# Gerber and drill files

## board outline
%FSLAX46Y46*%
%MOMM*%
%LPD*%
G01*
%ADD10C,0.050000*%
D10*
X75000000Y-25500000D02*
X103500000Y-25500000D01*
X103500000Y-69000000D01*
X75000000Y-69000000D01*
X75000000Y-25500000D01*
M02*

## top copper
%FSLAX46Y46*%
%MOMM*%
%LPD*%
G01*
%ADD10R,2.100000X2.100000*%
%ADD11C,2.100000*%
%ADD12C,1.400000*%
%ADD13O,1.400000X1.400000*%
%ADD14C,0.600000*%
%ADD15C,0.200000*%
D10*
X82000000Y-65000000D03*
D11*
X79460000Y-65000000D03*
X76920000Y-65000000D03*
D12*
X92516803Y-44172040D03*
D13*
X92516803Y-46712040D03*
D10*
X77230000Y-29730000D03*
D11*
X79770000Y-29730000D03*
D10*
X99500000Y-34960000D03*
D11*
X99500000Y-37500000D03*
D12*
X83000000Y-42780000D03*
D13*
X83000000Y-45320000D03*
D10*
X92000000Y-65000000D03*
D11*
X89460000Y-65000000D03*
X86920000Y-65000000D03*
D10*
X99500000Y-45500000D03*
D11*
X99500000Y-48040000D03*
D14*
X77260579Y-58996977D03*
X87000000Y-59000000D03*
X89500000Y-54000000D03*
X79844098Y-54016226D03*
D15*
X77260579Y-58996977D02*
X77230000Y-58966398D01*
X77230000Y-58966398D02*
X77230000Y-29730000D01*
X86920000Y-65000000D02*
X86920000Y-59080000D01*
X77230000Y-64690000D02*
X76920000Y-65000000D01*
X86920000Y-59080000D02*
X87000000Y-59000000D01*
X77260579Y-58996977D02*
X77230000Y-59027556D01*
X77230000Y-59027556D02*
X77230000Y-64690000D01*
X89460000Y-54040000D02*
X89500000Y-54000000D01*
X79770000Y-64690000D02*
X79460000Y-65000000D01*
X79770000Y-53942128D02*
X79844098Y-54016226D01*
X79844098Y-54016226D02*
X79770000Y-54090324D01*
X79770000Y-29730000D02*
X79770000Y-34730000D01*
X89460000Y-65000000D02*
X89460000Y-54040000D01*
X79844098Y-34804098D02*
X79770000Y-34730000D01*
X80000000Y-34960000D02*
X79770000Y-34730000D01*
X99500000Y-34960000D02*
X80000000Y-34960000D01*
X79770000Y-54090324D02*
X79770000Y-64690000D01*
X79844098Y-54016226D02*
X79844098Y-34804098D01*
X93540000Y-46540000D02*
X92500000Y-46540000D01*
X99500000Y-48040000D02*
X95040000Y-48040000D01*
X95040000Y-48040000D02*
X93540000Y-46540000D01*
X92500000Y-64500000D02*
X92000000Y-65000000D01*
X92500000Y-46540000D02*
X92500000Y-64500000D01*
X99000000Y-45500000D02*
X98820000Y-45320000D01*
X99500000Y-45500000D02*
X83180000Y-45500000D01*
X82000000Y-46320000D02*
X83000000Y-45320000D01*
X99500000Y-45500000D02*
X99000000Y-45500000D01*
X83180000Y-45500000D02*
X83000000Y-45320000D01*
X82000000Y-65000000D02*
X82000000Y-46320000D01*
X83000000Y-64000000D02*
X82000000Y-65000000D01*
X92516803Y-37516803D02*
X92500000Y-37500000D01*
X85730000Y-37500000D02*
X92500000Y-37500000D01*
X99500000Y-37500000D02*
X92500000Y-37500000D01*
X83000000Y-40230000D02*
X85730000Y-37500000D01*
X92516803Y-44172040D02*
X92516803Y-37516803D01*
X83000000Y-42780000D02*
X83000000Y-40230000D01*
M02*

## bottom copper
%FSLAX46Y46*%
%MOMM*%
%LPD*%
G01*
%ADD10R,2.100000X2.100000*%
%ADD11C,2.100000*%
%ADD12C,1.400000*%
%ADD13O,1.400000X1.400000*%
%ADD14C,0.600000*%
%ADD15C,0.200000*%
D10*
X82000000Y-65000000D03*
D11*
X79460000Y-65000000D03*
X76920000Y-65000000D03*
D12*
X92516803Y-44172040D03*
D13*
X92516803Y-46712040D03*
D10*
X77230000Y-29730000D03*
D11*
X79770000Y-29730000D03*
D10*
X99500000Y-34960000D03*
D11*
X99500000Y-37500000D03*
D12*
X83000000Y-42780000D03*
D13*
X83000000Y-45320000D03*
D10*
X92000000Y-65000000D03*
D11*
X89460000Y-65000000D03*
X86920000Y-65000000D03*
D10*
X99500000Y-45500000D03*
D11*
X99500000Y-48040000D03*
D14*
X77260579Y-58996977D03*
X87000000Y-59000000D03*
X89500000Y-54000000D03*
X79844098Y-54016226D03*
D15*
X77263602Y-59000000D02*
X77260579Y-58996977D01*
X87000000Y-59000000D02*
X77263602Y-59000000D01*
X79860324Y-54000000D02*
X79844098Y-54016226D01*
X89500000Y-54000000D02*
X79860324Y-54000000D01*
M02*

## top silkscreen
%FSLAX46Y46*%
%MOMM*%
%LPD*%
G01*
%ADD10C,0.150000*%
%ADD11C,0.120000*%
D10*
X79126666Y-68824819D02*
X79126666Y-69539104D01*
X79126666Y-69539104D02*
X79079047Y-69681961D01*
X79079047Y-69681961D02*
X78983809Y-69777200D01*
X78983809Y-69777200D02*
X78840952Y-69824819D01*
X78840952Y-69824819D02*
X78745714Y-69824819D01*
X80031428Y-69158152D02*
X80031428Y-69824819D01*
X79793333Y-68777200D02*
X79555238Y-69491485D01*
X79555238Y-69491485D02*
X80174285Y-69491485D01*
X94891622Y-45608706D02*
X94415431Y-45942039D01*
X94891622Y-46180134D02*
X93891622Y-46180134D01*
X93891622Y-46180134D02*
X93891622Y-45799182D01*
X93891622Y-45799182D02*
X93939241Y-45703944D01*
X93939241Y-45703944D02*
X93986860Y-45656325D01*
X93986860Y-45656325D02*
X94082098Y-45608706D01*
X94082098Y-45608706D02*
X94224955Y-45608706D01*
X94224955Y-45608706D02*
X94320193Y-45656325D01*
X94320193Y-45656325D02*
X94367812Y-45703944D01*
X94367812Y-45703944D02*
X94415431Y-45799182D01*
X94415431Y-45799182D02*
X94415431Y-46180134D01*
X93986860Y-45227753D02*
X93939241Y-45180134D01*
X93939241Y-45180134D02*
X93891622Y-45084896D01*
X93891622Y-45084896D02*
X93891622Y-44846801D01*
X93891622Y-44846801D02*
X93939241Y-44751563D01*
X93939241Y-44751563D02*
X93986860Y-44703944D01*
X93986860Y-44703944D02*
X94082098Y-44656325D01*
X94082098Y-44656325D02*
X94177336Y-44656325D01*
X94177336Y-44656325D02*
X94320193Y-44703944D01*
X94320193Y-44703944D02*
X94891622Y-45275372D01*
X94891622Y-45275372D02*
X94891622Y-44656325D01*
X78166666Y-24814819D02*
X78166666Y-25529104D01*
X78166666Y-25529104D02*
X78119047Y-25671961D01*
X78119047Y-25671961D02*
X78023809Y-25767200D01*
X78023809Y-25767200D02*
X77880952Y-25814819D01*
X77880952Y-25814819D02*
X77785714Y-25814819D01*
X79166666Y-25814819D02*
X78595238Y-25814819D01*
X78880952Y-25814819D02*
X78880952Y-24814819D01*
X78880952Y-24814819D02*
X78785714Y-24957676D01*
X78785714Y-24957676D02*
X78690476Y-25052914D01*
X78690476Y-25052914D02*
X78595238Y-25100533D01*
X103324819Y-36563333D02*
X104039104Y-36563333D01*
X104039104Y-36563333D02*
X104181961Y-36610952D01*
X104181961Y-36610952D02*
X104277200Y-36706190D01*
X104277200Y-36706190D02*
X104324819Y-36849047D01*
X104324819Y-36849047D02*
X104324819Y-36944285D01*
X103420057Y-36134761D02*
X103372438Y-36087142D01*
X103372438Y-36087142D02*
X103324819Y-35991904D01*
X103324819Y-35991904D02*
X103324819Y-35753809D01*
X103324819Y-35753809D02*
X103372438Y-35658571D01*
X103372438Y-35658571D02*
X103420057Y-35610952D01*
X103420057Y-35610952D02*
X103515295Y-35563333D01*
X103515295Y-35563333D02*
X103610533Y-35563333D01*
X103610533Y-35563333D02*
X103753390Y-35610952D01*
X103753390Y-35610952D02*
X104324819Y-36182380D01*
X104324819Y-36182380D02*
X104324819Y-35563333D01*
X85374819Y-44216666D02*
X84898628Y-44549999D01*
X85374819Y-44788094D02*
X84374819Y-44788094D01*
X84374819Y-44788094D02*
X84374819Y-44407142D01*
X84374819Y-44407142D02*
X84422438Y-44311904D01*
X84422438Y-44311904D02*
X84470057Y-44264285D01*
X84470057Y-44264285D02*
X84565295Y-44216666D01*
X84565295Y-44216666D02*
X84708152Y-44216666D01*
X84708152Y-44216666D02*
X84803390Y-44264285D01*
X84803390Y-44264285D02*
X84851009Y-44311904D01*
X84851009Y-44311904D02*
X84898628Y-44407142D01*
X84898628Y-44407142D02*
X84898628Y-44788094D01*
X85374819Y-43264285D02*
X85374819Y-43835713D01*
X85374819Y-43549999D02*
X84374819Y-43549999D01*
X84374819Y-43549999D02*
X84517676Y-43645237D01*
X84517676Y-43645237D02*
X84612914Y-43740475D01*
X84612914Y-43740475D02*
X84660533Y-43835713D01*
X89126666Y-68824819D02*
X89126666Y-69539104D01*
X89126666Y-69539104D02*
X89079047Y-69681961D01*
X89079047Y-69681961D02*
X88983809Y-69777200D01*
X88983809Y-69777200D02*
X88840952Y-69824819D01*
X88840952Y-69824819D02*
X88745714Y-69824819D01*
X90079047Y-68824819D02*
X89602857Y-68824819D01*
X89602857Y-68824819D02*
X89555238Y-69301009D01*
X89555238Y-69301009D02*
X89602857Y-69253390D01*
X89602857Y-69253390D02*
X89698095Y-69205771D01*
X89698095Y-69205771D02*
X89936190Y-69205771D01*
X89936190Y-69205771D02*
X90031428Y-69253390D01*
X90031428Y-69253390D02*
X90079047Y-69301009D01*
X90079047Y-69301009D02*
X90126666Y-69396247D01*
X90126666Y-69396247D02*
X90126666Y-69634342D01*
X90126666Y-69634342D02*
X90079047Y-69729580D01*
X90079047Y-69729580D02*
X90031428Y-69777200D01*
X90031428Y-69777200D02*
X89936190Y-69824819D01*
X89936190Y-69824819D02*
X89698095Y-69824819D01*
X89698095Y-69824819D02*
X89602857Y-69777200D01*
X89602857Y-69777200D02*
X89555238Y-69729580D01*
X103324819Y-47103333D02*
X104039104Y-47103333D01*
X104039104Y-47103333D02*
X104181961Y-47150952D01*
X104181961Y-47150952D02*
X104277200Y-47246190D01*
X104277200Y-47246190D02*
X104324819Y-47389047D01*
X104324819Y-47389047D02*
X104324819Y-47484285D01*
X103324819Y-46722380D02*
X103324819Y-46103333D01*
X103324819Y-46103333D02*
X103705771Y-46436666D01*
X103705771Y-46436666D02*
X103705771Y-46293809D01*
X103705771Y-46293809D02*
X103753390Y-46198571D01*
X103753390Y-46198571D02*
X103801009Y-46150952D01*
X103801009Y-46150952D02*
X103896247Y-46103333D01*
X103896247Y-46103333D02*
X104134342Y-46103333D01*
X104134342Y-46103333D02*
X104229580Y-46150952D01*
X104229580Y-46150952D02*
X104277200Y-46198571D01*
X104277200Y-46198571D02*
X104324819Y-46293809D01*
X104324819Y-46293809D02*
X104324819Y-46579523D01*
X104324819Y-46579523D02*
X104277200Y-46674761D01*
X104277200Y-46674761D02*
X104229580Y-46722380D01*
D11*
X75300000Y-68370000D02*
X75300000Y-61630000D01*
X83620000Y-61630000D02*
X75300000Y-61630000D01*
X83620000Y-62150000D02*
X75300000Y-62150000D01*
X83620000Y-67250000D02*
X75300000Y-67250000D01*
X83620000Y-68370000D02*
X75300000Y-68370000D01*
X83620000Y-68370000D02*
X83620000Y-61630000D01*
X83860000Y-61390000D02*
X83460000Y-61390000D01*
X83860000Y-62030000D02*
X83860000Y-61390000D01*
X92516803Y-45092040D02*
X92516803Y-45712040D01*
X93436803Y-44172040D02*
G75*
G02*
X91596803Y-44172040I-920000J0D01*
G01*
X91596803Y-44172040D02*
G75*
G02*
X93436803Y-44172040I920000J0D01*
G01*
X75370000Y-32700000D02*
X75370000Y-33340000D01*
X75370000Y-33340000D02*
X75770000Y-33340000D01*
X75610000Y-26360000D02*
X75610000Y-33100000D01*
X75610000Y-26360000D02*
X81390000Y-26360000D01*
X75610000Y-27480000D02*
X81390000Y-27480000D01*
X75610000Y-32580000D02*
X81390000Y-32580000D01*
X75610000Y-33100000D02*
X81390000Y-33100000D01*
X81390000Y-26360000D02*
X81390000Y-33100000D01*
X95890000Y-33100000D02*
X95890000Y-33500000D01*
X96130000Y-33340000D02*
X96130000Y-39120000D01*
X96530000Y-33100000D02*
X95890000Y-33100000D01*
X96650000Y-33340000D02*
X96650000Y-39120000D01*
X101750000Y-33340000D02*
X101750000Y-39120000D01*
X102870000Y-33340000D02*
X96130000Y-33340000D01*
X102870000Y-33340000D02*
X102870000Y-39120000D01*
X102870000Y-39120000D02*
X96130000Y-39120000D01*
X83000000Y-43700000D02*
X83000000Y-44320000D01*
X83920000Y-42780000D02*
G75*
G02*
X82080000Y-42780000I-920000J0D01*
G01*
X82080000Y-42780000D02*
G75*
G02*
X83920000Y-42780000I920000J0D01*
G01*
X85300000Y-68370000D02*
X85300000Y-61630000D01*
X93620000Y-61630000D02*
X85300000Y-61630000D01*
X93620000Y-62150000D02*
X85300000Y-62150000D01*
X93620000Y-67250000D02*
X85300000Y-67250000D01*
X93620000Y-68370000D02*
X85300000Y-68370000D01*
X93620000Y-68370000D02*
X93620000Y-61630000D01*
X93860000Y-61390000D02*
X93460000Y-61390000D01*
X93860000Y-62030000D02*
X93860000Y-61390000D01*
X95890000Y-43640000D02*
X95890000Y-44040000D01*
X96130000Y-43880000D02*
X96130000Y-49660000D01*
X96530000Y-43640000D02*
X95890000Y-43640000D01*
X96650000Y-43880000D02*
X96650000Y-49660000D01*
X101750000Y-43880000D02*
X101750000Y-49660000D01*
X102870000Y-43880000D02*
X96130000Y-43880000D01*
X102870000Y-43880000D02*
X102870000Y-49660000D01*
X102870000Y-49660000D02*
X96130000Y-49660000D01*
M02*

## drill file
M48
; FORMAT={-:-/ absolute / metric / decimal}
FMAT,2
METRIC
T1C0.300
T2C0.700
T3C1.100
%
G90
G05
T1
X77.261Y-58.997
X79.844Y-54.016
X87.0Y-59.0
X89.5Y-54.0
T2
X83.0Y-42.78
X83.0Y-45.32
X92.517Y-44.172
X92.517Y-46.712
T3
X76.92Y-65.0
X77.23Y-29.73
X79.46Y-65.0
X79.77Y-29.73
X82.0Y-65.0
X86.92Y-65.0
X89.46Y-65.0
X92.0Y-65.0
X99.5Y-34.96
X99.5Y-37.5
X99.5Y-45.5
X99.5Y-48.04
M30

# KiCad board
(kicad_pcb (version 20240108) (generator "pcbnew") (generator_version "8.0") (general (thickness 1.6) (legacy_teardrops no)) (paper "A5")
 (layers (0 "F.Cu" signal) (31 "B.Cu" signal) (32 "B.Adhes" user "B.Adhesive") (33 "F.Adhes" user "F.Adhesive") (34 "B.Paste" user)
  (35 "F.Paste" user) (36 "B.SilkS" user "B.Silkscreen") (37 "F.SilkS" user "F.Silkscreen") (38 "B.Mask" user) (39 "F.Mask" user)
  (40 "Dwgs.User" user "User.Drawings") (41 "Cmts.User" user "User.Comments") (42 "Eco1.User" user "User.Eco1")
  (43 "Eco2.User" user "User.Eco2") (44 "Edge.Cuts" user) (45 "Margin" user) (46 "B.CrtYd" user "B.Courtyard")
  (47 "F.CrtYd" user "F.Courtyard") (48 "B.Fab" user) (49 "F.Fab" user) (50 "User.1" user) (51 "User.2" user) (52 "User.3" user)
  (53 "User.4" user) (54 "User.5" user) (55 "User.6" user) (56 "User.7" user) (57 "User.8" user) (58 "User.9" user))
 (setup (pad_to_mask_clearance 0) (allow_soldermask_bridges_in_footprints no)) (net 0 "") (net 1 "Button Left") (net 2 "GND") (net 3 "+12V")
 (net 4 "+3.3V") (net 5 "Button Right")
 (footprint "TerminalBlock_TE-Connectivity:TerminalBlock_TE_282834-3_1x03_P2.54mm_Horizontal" (layer "F.Cu") (at 82 65 180)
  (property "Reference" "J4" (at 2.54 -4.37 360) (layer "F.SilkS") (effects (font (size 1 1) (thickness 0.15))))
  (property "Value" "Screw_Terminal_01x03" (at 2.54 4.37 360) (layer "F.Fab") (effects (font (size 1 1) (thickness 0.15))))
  (fp_line (start 6.7 -3.37) (end 6.7 3.37) (stroke (width 0.12) (type solid)) (layer "F.SilkS"))
  (fp_line (start -1.62 3.37) (end 6.7 3.37) (stroke (width 0.12) (type solid)) (layer "F.SilkS"))
  (fp_line (start -1.62 2.85) (end 6.7 2.85) (stroke (width 0.12) (type solid)) (layer "F.SilkS"))
  (fp_line (start -1.62 -2.25) (end 6.7 -2.25) (stroke (width 0.12) (type solid)) (layer "F.SilkS"))
  (fp_line (start -1.62 -3.37) (end 6.7 -3.37) (stroke (width 0.12) (type solid)) (layer "F.SilkS"))
  (fp_line (start -1.62 -3.37) (end -1.62 3.37) (stroke (width 0.12) (type solid)) (layer "F.SilkS"))
  (fp_line (start -1.86 3.61) (end -1.46 3.61) (stroke (width 0.12) (type solid)) (layer "F.SilkS"))
  (fp_line (start -1.86 2.97) (end -1.86 3.61) (stroke (width 0.12) (type solid)) (layer "F.SilkS"))
  (pad "1" thru_hole rect (at 0 0 180) (size 2.1 2.1) (drill 1.1) (layers "*.Cu" "*.Mask") (remove_unused_layers no) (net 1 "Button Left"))
  (pad "2" thru_hole circle (at 2.54 0 180) (size 2.1 2.1) (drill 1.1) (layers "*.Cu" "*.Mask") (remove_unused_layers no) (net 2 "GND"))
  (pad "3" thru_hole circle (at 5.08 0 180) (size 2.1 2.1) (drill 1.1) (layers "*.Cu" "*.Mask") (remove_unused_layers no) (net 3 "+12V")))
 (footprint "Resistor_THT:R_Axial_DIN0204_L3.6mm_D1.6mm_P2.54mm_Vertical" (layer "F.Cu") (at 92.516803 44.17204 -90)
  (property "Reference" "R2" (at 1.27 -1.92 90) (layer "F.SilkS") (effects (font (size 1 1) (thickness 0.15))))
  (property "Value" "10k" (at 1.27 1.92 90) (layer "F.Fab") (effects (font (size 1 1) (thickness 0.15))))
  (fp_line (start 0.92 0) (end 1.54 0) (stroke (width 0.12) (type solid)) (layer "F.SilkS"))
  (fp_circle (center 0 0) (end 0.92 0) (stroke (width 0.12) (type solid)) (fill none) (layer "F.SilkS"))
  (pad "1" thru_hole circle (at 0 0 270) (size 1.4 1.4) (drill 0.7) (layers "*.Cu" "*.Mask") (remove_unused_layers no) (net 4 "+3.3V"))
  (pad "2" thru_hole oval (at 2.54 0 270) (size 1.4 1.4) (drill 0.7) (layers "*.Cu" "*.Mask") (remove_unused_layers no)
   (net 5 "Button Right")))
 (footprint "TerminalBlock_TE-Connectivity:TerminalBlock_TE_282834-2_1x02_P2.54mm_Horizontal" (layer "F.Cu") (at 77.23 29.73)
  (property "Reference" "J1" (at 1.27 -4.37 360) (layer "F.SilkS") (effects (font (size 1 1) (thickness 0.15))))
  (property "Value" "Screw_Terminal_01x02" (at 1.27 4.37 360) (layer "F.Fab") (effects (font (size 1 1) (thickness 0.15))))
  (fp_line (start -1.86 2.97) (end -1.86 3.61) (stroke (width 0.12) (type solid)) (layer "F.SilkS"))
  (fp_line (start -1.86 3.61) (end -1.46 3.61) (stroke (width 0.12) (type solid)) (layer "F.SilkS"))
  (fp_line (start -1.62 -3.37) (end -1.62 3.37) (stroke (width 0.12) (type solid)) (layer "F.SilkS"))
  (fp_line (start -1.62 -3.37) (end 4.16 -3.37) (stroke (width 0.12) (type solid)) (layer "F.SilkS"))
  (fp_line (start -1.62 -2.25) (end 4.16 -2.25) (stroke (width 0.12) (type solid)) (layer "F.SilkS"))
  (fp_line (start -1.62 2.85) (end 4.16 2.85) (stroke (width 0.12) (type solid)) (layer "F.SilkS"))
  (fp_line (start -1.62 3.37) (end 4.16 3.37) (stroke (width 0.12) (type solid)) (layer "F.SilkS"))
  (fp_line (start 4.16 -3.37) (end 4.16 3.37) (stroke (width 0.12) (type solid)) (layer "F.SilkS"))
  (pad "1" thru_hole rect (at 0 0) (size 2.1 2.1) (drill 1.1) (layers "*.Cu" "*.Mask") (remove_unused_layers no) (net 3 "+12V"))
  (pad "2" thru_hole circle (at 2.54 0) (size 2.1 2.1) (drill 1.1) (layers "*.Cu" "*.Mask") (remove_unused_layers no) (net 2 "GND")))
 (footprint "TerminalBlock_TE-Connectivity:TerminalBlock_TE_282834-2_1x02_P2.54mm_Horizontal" (layer "F.Cu") (at 99.5 34.96 -90)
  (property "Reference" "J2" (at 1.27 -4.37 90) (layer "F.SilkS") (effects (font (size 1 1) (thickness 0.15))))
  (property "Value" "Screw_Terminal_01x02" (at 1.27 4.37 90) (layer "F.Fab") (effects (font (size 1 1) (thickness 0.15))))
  (fp_line (start -1.86 3.61) (end -1.46 3.61) (stroke (width 0.12) (type solid)) (layer "F.SilkS"))
  (fp_line (start -1.62 3.37) (end 4.16 3.37) (stroke (width 0.12) (type solid)) (layer "F.SilkS"))
  (fp_line (start -1.86 2.97) (end -1.86 3.61) (stroke (width 0.12) (type solid)) (layer "F.SilkS"))
  (fp_line (start -1.62 2.85) (end 4.16 2.85) (stroke (width 0.12) (type solid)) (layer "F.SilkS"))
  (fp_line (start -1.62 -2.25) (end 4.16 -2.25) (stroke (width 0.12) (type solid)) (layer "F.SilkS"))
  (fp_line (start -1.62 -3.37) (end -1.62 3.37) (stroke (width 0.12) (type solid)) (layer "F.SilkS"))
  (fp_line (start -1.62 -3.37) (end 4.16 -3.37) (stroke (width 0.12) (type solid)) (layer "F.SilkS"))
  (fp_line (start 4.16 -3.37) (end 4.16 3.37) (stroke (width 0.12) (type solid)) (layer "F.SilkS"))
  (pad "1" thru_hole rect (at 0 0 270) (size 2.1 2.1) (drill 1.1) (layers "*.Cu" "*.Mask") (remove_unused_layers no) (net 2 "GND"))
  (pad "2" thru_hole circle (at 2.54 0 270) (size 2.1 2.1) (drill 1.1) (layers "*.Cu" "*.Mask") (remove_unused_layers no) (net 4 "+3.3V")))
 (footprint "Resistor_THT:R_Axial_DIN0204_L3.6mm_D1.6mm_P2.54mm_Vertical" (layer "F.Cu") (at 83 42.78 -90)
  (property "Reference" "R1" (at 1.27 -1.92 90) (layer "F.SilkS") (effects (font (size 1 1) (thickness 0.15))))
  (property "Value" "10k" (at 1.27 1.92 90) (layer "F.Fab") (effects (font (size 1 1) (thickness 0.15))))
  (fp_line (start 0.92 0) (end 1.54 0) (stroke (width 0.12) (type solid)) (layer "F.SilkS"))
  (fp_circle (center 0 0) (end 0.92 0) (stroke (width 0.12) (type solid)) (fill none) (layer "F.SilkS"))
  (pad "1" thru_hole circle (at 0 0 270) (size 1.4 1.4) (drill 0.7) (layers "*.Cu" "*.Mask") (remove_unused_layers no) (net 4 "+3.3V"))
  (pad "2" thru_hole oval (at 2.54 0 270) (size 1.4 1.4) (drill 0.7) (layers "*.Cu" "*.Mask") (remove_unused_layers no)
   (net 1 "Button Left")))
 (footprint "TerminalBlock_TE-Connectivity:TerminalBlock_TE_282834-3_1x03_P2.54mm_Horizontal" (layer "F.Cu") (at 92 65 180)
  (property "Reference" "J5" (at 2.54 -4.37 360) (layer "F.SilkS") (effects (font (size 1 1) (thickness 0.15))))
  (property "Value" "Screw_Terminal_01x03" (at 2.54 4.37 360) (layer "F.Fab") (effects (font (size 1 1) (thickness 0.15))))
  (fp_line (start 6.7 -3.37) (end 6.7 3.37) (stroke (width 0.12) (type solid)) (layer "F.SilkS"))
  (fp_line (start -1.62 3.37) (end 6.7 3.37) (stroke (width 0.12) (type solid)) (layer "F.SilkS"))
  (fp_line (start -1.62 2.85) (end 6.7 2.85) (stroke (width 0.12) (type solid)) (layer "F.SilkS"))
  (fp_line (start -1.62 -2.25) (end 6.7 -2.25) (stroke (width 0.12) (type solid)) (layer "F.SilkS"))
  (fp_line (start -1.62 -3.37) (end 6.7 -3.37) (stroke (width 0.12) (type solid)) (layer "F.SilkS"))
  (fp_line (start -1.62 -3.37) (end -1.62 3.37) (stroke (width 0.12) (type solid)) (layer "F.SilkS"))
  (fp_line (start -1.86 3.61) (end -1.46 3.61) (stroke (width 0.12) (type solid)) (layer "F.SilkS"))
  (fp_line (start -1.86 2.97) (end -1.86 3.61) (stroke (width 0.12) (type solid)) (layer "F.SilkS"))
  (pad "1" thru_hole rect (at 0 0 180) (size 2.1 2.1) (drill 1.1) (layers "*.Cu" "*.Mask") (remove_unused_layers no) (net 5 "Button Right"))
  (pad "2" thru_hole circle (at 2.54 0 180) (size 2.1 2.1) (drill 1.1) (layers "*.Cu" "*.Mask") (remove_unused_layers no) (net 2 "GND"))
  (pad "3" thru_hole circle (at 5.08 0 180) (size 2.1 2.1) (drill 1.1) (layers "*.Cu" "*.Mask") (remove_unused_layers no) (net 3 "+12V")))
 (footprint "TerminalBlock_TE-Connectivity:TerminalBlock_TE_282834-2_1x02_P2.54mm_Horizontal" (layer "F.Cu") (at 99.5 45.5 -90)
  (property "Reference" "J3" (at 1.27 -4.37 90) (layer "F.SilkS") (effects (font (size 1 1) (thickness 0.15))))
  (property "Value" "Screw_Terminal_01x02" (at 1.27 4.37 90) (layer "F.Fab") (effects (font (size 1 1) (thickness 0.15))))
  (fp_line (start -1.86 3.61) (end -1.46 3.61) (stroke (width 0.12) (type solid)) (layer "F.SilkS"))
  (fp_line (start -1.62 3.37) (end 4.16 3.37) (stroke (width 0.12) (type solid)) (layer "F.SilkS"))
  (fp_line (start -1.86 2.97) (end -1.86 3.61) (stroke (width 0.12) (type solid)) (layer "F.SilkS"))
  (fp_line (start -1.62 2.85) (end 4.16 2.85) (stroke (width 0.12) (type solid)) (layer "F.SilkS"))
  (fp_line (start -1.62 -2.25) (end 4.16 -2.25) (stroke (width 0.12) (type solid)) (layer "F.SilkS"))
  (fp_line (start -1.62 -3.37) (end -1.62 3.37) (stroke (width 0.12) (type solid)) (layer "F.SilkS"))
  (fp_line (start -1.62 -3.37) (end 4.16 -3.37) (stroke (width 0.12) (type solid)) (layer "F.SilkS"))
  (fp_line (start 4.16 -3.37) (end 4.16 3.37) (stroke (width 0.12) (type solid)) (layer "F.SilkS"))
  (pad "1" thru_hole rect (at 0 0 270) (size 2.1 2.1) (drill 1.1) (layers "*.Cu" "*.Mask") (remove_unused_layers no) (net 1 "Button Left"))
  (pad "2" thru_hole circle (at 2.54 0 270) (size 2.1 2.1) (drill 1.1) (layers "*.Cu" "*.Mask") (remove_unused_layers no)
   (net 5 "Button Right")))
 (gr_rect (start 75 25.5) (end 103.5 69) (stroke (width 0.05) (type default)) (fill none) (layer "Edge.Cuts"))
 (segment (start 77.260579 58.996977) (end 77.23 58.966398) (width 0.2) (layer "F.Cu") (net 3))
 (segment (start 77.23 58.966398) (end 77.23 29.73) (width 0.2) (layer "F.Cu") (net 3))
 (segment (start 86.92 65) (end 86.92 59.08) (width 0.2) (layer "F.Cu") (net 3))
 (segment (start 77.23 64.69) (end 76.92 65) (width 0.2) (layer "F.Cu") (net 3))
 (segment (start 86.92 59.08) (end 87 59) (width 0.2) (layer "F.Cu") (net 3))
 (segment (start 77.260579 58.996977) (end 77.23 59.027556) (width 0.2) (layer "F.Cu") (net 3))
 (segment (start 77.23 59.027556) (end 77.23 64.69) (width 0.2) (layer "F.Cu") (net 3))
 (via (at 77.260579 58.996977) (size 0.6) (drill 0.3) (layers "F.Cu" "B.Cu") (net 3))
 (via (at 87 59) (size 0.6) (drill 0.3) (layers "F.Cu" "B.Cu") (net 3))
 (segment (start 77.263602 59) (end 77.260579 58.996977) (width 0.2) (layer "B.Cu") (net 3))
 (segment (start 87 59) (end 77.263602 59) (width 0.2) (layer "B.Cu") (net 3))
 (segment (start 89.46 54.04) (end 89.5 54) (width 0.2) (layer "F.Cu") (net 2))
 (segment (start 79.77 64.69) (end 79.46 65) (width 0.2) (layer "F.Cu") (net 2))
 (segment (start 79.77 53.942128) (end 79.844098 54.016226) (width 0.2) (layer "F.Cu") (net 2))
 (segment (start 79.844098 54.016226) (end 79.77 54.090324) (width 0.2) (layer "F.Cu") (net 2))
 (segment (start 79.77 29.73) (end 79.77 34.73) (width 0.2) (layer "F.Cu") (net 2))
 (segment (start 89.46 65) (end 89.46 54.04) (width 0.2) (layer "F.Cu") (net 2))
 (segment (start 79.844098 34.804098) (end 79.77 34.73) (width 0.2) (layer "F.Cu") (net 2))
 (segment (start 80 34.96) (end 79.77 34.73) (width 0.2) (layer "F.Cu") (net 2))
 (segment (start 99.5 34.96) (end 80 34.96) (width 0.2) (layer "F.Cu") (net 2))
 (segment (start 79.77 54.090324) (end 79.77 64.69) (width 0.2) (layer "F.Cu") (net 2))
 (segment (start 79.844098 54.016226) (end 79.844098 34.804098) (width 0.2) (layer "F.Cu") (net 2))
 (via (at 89.5 54) (size 0.6) (drill 0.3) (layers "F.Cu" "B.Cu") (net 2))
 (via (at 79.844098 54.016226) (size 0.6) (drill 0.3) (layers "F.Cu" "B.Cu") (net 2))
 (segment (start 79.860324 54) (end 79.844098 54.016226) (width 0.2) (layer "B.Cu") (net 2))
 (segment (start 89.5 54) (end 79.860324 54) (width 0.2) (layer "B.Cu") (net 2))
 (segment (start 93.54 46.54) (end 92.5 46.54) (width 0.2) (layer "F.Cu") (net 5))
 (segment (start 99.5 48.04) (end 95.04 48.04) (width 0.2) (layer "F.Cu") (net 5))
 (segment (start 95.04 48.04) (end 93.54 46.54) (width 0.2) (layer "F.Cu") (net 5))
 (segment (start 92.5 64.5) (end 92 65) (width 0.2) (layer "F.Cu") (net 5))
 (segment (start 92.5 46.54) (end 92.5 64.5) (width 0.2) (layer "F.Cu") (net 5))
 (segment (start 99 45.5) (end 98.82 45.32) (width 0.2) (layer "F.Cu") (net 1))
 (segment (start 99.5 45.5) (end 83.18 45.5) (width 0.2) (layer "F.Cu") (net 1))
 (segment (start 82 46.32) (end 83 45.32) (width 0.2) (layer "F.Cu") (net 1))
 (segment (start 99.5 45.5) (end 99 45.5) (width 0.2) (layer "F.Cu") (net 1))
 (segment (start 83.18 45.5) (end 83 45.32) (width 0.2) (layer "F.Cu") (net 1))
 (segment (start 82 65) (end 82 46.32) (width 0.2) (layer "F.Cu") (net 1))
 (segment (start 83 64) (end 82 65) (width 0.2) (layer "F.Cu") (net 1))
 (segment (start 92.516803 37.516803) (end 92.5 37.5) (width 0.2) (layer "F.Cu") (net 4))
 (segment (start 85.73 37.5) (end 92.5 37.5) (width 0.2) (layer "F.Cu") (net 4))
 (segment (start 99.5 37.5) (end 92.5 37.5) (width 0.2) (layer "F.Cu") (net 4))
 (segment (start 83 40.23) (end 85.73 37.5) (width 0.2) (layer "F.Cu") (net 4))
 (segment (start 92.516803 44.17204) (end 92.516803 37.516803) (width 0.2) (layer "F.Cu") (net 4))
 (segment (start 83 42.78) (end 83 40.23) (width 0.2) (layer "F.Cu") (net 4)))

